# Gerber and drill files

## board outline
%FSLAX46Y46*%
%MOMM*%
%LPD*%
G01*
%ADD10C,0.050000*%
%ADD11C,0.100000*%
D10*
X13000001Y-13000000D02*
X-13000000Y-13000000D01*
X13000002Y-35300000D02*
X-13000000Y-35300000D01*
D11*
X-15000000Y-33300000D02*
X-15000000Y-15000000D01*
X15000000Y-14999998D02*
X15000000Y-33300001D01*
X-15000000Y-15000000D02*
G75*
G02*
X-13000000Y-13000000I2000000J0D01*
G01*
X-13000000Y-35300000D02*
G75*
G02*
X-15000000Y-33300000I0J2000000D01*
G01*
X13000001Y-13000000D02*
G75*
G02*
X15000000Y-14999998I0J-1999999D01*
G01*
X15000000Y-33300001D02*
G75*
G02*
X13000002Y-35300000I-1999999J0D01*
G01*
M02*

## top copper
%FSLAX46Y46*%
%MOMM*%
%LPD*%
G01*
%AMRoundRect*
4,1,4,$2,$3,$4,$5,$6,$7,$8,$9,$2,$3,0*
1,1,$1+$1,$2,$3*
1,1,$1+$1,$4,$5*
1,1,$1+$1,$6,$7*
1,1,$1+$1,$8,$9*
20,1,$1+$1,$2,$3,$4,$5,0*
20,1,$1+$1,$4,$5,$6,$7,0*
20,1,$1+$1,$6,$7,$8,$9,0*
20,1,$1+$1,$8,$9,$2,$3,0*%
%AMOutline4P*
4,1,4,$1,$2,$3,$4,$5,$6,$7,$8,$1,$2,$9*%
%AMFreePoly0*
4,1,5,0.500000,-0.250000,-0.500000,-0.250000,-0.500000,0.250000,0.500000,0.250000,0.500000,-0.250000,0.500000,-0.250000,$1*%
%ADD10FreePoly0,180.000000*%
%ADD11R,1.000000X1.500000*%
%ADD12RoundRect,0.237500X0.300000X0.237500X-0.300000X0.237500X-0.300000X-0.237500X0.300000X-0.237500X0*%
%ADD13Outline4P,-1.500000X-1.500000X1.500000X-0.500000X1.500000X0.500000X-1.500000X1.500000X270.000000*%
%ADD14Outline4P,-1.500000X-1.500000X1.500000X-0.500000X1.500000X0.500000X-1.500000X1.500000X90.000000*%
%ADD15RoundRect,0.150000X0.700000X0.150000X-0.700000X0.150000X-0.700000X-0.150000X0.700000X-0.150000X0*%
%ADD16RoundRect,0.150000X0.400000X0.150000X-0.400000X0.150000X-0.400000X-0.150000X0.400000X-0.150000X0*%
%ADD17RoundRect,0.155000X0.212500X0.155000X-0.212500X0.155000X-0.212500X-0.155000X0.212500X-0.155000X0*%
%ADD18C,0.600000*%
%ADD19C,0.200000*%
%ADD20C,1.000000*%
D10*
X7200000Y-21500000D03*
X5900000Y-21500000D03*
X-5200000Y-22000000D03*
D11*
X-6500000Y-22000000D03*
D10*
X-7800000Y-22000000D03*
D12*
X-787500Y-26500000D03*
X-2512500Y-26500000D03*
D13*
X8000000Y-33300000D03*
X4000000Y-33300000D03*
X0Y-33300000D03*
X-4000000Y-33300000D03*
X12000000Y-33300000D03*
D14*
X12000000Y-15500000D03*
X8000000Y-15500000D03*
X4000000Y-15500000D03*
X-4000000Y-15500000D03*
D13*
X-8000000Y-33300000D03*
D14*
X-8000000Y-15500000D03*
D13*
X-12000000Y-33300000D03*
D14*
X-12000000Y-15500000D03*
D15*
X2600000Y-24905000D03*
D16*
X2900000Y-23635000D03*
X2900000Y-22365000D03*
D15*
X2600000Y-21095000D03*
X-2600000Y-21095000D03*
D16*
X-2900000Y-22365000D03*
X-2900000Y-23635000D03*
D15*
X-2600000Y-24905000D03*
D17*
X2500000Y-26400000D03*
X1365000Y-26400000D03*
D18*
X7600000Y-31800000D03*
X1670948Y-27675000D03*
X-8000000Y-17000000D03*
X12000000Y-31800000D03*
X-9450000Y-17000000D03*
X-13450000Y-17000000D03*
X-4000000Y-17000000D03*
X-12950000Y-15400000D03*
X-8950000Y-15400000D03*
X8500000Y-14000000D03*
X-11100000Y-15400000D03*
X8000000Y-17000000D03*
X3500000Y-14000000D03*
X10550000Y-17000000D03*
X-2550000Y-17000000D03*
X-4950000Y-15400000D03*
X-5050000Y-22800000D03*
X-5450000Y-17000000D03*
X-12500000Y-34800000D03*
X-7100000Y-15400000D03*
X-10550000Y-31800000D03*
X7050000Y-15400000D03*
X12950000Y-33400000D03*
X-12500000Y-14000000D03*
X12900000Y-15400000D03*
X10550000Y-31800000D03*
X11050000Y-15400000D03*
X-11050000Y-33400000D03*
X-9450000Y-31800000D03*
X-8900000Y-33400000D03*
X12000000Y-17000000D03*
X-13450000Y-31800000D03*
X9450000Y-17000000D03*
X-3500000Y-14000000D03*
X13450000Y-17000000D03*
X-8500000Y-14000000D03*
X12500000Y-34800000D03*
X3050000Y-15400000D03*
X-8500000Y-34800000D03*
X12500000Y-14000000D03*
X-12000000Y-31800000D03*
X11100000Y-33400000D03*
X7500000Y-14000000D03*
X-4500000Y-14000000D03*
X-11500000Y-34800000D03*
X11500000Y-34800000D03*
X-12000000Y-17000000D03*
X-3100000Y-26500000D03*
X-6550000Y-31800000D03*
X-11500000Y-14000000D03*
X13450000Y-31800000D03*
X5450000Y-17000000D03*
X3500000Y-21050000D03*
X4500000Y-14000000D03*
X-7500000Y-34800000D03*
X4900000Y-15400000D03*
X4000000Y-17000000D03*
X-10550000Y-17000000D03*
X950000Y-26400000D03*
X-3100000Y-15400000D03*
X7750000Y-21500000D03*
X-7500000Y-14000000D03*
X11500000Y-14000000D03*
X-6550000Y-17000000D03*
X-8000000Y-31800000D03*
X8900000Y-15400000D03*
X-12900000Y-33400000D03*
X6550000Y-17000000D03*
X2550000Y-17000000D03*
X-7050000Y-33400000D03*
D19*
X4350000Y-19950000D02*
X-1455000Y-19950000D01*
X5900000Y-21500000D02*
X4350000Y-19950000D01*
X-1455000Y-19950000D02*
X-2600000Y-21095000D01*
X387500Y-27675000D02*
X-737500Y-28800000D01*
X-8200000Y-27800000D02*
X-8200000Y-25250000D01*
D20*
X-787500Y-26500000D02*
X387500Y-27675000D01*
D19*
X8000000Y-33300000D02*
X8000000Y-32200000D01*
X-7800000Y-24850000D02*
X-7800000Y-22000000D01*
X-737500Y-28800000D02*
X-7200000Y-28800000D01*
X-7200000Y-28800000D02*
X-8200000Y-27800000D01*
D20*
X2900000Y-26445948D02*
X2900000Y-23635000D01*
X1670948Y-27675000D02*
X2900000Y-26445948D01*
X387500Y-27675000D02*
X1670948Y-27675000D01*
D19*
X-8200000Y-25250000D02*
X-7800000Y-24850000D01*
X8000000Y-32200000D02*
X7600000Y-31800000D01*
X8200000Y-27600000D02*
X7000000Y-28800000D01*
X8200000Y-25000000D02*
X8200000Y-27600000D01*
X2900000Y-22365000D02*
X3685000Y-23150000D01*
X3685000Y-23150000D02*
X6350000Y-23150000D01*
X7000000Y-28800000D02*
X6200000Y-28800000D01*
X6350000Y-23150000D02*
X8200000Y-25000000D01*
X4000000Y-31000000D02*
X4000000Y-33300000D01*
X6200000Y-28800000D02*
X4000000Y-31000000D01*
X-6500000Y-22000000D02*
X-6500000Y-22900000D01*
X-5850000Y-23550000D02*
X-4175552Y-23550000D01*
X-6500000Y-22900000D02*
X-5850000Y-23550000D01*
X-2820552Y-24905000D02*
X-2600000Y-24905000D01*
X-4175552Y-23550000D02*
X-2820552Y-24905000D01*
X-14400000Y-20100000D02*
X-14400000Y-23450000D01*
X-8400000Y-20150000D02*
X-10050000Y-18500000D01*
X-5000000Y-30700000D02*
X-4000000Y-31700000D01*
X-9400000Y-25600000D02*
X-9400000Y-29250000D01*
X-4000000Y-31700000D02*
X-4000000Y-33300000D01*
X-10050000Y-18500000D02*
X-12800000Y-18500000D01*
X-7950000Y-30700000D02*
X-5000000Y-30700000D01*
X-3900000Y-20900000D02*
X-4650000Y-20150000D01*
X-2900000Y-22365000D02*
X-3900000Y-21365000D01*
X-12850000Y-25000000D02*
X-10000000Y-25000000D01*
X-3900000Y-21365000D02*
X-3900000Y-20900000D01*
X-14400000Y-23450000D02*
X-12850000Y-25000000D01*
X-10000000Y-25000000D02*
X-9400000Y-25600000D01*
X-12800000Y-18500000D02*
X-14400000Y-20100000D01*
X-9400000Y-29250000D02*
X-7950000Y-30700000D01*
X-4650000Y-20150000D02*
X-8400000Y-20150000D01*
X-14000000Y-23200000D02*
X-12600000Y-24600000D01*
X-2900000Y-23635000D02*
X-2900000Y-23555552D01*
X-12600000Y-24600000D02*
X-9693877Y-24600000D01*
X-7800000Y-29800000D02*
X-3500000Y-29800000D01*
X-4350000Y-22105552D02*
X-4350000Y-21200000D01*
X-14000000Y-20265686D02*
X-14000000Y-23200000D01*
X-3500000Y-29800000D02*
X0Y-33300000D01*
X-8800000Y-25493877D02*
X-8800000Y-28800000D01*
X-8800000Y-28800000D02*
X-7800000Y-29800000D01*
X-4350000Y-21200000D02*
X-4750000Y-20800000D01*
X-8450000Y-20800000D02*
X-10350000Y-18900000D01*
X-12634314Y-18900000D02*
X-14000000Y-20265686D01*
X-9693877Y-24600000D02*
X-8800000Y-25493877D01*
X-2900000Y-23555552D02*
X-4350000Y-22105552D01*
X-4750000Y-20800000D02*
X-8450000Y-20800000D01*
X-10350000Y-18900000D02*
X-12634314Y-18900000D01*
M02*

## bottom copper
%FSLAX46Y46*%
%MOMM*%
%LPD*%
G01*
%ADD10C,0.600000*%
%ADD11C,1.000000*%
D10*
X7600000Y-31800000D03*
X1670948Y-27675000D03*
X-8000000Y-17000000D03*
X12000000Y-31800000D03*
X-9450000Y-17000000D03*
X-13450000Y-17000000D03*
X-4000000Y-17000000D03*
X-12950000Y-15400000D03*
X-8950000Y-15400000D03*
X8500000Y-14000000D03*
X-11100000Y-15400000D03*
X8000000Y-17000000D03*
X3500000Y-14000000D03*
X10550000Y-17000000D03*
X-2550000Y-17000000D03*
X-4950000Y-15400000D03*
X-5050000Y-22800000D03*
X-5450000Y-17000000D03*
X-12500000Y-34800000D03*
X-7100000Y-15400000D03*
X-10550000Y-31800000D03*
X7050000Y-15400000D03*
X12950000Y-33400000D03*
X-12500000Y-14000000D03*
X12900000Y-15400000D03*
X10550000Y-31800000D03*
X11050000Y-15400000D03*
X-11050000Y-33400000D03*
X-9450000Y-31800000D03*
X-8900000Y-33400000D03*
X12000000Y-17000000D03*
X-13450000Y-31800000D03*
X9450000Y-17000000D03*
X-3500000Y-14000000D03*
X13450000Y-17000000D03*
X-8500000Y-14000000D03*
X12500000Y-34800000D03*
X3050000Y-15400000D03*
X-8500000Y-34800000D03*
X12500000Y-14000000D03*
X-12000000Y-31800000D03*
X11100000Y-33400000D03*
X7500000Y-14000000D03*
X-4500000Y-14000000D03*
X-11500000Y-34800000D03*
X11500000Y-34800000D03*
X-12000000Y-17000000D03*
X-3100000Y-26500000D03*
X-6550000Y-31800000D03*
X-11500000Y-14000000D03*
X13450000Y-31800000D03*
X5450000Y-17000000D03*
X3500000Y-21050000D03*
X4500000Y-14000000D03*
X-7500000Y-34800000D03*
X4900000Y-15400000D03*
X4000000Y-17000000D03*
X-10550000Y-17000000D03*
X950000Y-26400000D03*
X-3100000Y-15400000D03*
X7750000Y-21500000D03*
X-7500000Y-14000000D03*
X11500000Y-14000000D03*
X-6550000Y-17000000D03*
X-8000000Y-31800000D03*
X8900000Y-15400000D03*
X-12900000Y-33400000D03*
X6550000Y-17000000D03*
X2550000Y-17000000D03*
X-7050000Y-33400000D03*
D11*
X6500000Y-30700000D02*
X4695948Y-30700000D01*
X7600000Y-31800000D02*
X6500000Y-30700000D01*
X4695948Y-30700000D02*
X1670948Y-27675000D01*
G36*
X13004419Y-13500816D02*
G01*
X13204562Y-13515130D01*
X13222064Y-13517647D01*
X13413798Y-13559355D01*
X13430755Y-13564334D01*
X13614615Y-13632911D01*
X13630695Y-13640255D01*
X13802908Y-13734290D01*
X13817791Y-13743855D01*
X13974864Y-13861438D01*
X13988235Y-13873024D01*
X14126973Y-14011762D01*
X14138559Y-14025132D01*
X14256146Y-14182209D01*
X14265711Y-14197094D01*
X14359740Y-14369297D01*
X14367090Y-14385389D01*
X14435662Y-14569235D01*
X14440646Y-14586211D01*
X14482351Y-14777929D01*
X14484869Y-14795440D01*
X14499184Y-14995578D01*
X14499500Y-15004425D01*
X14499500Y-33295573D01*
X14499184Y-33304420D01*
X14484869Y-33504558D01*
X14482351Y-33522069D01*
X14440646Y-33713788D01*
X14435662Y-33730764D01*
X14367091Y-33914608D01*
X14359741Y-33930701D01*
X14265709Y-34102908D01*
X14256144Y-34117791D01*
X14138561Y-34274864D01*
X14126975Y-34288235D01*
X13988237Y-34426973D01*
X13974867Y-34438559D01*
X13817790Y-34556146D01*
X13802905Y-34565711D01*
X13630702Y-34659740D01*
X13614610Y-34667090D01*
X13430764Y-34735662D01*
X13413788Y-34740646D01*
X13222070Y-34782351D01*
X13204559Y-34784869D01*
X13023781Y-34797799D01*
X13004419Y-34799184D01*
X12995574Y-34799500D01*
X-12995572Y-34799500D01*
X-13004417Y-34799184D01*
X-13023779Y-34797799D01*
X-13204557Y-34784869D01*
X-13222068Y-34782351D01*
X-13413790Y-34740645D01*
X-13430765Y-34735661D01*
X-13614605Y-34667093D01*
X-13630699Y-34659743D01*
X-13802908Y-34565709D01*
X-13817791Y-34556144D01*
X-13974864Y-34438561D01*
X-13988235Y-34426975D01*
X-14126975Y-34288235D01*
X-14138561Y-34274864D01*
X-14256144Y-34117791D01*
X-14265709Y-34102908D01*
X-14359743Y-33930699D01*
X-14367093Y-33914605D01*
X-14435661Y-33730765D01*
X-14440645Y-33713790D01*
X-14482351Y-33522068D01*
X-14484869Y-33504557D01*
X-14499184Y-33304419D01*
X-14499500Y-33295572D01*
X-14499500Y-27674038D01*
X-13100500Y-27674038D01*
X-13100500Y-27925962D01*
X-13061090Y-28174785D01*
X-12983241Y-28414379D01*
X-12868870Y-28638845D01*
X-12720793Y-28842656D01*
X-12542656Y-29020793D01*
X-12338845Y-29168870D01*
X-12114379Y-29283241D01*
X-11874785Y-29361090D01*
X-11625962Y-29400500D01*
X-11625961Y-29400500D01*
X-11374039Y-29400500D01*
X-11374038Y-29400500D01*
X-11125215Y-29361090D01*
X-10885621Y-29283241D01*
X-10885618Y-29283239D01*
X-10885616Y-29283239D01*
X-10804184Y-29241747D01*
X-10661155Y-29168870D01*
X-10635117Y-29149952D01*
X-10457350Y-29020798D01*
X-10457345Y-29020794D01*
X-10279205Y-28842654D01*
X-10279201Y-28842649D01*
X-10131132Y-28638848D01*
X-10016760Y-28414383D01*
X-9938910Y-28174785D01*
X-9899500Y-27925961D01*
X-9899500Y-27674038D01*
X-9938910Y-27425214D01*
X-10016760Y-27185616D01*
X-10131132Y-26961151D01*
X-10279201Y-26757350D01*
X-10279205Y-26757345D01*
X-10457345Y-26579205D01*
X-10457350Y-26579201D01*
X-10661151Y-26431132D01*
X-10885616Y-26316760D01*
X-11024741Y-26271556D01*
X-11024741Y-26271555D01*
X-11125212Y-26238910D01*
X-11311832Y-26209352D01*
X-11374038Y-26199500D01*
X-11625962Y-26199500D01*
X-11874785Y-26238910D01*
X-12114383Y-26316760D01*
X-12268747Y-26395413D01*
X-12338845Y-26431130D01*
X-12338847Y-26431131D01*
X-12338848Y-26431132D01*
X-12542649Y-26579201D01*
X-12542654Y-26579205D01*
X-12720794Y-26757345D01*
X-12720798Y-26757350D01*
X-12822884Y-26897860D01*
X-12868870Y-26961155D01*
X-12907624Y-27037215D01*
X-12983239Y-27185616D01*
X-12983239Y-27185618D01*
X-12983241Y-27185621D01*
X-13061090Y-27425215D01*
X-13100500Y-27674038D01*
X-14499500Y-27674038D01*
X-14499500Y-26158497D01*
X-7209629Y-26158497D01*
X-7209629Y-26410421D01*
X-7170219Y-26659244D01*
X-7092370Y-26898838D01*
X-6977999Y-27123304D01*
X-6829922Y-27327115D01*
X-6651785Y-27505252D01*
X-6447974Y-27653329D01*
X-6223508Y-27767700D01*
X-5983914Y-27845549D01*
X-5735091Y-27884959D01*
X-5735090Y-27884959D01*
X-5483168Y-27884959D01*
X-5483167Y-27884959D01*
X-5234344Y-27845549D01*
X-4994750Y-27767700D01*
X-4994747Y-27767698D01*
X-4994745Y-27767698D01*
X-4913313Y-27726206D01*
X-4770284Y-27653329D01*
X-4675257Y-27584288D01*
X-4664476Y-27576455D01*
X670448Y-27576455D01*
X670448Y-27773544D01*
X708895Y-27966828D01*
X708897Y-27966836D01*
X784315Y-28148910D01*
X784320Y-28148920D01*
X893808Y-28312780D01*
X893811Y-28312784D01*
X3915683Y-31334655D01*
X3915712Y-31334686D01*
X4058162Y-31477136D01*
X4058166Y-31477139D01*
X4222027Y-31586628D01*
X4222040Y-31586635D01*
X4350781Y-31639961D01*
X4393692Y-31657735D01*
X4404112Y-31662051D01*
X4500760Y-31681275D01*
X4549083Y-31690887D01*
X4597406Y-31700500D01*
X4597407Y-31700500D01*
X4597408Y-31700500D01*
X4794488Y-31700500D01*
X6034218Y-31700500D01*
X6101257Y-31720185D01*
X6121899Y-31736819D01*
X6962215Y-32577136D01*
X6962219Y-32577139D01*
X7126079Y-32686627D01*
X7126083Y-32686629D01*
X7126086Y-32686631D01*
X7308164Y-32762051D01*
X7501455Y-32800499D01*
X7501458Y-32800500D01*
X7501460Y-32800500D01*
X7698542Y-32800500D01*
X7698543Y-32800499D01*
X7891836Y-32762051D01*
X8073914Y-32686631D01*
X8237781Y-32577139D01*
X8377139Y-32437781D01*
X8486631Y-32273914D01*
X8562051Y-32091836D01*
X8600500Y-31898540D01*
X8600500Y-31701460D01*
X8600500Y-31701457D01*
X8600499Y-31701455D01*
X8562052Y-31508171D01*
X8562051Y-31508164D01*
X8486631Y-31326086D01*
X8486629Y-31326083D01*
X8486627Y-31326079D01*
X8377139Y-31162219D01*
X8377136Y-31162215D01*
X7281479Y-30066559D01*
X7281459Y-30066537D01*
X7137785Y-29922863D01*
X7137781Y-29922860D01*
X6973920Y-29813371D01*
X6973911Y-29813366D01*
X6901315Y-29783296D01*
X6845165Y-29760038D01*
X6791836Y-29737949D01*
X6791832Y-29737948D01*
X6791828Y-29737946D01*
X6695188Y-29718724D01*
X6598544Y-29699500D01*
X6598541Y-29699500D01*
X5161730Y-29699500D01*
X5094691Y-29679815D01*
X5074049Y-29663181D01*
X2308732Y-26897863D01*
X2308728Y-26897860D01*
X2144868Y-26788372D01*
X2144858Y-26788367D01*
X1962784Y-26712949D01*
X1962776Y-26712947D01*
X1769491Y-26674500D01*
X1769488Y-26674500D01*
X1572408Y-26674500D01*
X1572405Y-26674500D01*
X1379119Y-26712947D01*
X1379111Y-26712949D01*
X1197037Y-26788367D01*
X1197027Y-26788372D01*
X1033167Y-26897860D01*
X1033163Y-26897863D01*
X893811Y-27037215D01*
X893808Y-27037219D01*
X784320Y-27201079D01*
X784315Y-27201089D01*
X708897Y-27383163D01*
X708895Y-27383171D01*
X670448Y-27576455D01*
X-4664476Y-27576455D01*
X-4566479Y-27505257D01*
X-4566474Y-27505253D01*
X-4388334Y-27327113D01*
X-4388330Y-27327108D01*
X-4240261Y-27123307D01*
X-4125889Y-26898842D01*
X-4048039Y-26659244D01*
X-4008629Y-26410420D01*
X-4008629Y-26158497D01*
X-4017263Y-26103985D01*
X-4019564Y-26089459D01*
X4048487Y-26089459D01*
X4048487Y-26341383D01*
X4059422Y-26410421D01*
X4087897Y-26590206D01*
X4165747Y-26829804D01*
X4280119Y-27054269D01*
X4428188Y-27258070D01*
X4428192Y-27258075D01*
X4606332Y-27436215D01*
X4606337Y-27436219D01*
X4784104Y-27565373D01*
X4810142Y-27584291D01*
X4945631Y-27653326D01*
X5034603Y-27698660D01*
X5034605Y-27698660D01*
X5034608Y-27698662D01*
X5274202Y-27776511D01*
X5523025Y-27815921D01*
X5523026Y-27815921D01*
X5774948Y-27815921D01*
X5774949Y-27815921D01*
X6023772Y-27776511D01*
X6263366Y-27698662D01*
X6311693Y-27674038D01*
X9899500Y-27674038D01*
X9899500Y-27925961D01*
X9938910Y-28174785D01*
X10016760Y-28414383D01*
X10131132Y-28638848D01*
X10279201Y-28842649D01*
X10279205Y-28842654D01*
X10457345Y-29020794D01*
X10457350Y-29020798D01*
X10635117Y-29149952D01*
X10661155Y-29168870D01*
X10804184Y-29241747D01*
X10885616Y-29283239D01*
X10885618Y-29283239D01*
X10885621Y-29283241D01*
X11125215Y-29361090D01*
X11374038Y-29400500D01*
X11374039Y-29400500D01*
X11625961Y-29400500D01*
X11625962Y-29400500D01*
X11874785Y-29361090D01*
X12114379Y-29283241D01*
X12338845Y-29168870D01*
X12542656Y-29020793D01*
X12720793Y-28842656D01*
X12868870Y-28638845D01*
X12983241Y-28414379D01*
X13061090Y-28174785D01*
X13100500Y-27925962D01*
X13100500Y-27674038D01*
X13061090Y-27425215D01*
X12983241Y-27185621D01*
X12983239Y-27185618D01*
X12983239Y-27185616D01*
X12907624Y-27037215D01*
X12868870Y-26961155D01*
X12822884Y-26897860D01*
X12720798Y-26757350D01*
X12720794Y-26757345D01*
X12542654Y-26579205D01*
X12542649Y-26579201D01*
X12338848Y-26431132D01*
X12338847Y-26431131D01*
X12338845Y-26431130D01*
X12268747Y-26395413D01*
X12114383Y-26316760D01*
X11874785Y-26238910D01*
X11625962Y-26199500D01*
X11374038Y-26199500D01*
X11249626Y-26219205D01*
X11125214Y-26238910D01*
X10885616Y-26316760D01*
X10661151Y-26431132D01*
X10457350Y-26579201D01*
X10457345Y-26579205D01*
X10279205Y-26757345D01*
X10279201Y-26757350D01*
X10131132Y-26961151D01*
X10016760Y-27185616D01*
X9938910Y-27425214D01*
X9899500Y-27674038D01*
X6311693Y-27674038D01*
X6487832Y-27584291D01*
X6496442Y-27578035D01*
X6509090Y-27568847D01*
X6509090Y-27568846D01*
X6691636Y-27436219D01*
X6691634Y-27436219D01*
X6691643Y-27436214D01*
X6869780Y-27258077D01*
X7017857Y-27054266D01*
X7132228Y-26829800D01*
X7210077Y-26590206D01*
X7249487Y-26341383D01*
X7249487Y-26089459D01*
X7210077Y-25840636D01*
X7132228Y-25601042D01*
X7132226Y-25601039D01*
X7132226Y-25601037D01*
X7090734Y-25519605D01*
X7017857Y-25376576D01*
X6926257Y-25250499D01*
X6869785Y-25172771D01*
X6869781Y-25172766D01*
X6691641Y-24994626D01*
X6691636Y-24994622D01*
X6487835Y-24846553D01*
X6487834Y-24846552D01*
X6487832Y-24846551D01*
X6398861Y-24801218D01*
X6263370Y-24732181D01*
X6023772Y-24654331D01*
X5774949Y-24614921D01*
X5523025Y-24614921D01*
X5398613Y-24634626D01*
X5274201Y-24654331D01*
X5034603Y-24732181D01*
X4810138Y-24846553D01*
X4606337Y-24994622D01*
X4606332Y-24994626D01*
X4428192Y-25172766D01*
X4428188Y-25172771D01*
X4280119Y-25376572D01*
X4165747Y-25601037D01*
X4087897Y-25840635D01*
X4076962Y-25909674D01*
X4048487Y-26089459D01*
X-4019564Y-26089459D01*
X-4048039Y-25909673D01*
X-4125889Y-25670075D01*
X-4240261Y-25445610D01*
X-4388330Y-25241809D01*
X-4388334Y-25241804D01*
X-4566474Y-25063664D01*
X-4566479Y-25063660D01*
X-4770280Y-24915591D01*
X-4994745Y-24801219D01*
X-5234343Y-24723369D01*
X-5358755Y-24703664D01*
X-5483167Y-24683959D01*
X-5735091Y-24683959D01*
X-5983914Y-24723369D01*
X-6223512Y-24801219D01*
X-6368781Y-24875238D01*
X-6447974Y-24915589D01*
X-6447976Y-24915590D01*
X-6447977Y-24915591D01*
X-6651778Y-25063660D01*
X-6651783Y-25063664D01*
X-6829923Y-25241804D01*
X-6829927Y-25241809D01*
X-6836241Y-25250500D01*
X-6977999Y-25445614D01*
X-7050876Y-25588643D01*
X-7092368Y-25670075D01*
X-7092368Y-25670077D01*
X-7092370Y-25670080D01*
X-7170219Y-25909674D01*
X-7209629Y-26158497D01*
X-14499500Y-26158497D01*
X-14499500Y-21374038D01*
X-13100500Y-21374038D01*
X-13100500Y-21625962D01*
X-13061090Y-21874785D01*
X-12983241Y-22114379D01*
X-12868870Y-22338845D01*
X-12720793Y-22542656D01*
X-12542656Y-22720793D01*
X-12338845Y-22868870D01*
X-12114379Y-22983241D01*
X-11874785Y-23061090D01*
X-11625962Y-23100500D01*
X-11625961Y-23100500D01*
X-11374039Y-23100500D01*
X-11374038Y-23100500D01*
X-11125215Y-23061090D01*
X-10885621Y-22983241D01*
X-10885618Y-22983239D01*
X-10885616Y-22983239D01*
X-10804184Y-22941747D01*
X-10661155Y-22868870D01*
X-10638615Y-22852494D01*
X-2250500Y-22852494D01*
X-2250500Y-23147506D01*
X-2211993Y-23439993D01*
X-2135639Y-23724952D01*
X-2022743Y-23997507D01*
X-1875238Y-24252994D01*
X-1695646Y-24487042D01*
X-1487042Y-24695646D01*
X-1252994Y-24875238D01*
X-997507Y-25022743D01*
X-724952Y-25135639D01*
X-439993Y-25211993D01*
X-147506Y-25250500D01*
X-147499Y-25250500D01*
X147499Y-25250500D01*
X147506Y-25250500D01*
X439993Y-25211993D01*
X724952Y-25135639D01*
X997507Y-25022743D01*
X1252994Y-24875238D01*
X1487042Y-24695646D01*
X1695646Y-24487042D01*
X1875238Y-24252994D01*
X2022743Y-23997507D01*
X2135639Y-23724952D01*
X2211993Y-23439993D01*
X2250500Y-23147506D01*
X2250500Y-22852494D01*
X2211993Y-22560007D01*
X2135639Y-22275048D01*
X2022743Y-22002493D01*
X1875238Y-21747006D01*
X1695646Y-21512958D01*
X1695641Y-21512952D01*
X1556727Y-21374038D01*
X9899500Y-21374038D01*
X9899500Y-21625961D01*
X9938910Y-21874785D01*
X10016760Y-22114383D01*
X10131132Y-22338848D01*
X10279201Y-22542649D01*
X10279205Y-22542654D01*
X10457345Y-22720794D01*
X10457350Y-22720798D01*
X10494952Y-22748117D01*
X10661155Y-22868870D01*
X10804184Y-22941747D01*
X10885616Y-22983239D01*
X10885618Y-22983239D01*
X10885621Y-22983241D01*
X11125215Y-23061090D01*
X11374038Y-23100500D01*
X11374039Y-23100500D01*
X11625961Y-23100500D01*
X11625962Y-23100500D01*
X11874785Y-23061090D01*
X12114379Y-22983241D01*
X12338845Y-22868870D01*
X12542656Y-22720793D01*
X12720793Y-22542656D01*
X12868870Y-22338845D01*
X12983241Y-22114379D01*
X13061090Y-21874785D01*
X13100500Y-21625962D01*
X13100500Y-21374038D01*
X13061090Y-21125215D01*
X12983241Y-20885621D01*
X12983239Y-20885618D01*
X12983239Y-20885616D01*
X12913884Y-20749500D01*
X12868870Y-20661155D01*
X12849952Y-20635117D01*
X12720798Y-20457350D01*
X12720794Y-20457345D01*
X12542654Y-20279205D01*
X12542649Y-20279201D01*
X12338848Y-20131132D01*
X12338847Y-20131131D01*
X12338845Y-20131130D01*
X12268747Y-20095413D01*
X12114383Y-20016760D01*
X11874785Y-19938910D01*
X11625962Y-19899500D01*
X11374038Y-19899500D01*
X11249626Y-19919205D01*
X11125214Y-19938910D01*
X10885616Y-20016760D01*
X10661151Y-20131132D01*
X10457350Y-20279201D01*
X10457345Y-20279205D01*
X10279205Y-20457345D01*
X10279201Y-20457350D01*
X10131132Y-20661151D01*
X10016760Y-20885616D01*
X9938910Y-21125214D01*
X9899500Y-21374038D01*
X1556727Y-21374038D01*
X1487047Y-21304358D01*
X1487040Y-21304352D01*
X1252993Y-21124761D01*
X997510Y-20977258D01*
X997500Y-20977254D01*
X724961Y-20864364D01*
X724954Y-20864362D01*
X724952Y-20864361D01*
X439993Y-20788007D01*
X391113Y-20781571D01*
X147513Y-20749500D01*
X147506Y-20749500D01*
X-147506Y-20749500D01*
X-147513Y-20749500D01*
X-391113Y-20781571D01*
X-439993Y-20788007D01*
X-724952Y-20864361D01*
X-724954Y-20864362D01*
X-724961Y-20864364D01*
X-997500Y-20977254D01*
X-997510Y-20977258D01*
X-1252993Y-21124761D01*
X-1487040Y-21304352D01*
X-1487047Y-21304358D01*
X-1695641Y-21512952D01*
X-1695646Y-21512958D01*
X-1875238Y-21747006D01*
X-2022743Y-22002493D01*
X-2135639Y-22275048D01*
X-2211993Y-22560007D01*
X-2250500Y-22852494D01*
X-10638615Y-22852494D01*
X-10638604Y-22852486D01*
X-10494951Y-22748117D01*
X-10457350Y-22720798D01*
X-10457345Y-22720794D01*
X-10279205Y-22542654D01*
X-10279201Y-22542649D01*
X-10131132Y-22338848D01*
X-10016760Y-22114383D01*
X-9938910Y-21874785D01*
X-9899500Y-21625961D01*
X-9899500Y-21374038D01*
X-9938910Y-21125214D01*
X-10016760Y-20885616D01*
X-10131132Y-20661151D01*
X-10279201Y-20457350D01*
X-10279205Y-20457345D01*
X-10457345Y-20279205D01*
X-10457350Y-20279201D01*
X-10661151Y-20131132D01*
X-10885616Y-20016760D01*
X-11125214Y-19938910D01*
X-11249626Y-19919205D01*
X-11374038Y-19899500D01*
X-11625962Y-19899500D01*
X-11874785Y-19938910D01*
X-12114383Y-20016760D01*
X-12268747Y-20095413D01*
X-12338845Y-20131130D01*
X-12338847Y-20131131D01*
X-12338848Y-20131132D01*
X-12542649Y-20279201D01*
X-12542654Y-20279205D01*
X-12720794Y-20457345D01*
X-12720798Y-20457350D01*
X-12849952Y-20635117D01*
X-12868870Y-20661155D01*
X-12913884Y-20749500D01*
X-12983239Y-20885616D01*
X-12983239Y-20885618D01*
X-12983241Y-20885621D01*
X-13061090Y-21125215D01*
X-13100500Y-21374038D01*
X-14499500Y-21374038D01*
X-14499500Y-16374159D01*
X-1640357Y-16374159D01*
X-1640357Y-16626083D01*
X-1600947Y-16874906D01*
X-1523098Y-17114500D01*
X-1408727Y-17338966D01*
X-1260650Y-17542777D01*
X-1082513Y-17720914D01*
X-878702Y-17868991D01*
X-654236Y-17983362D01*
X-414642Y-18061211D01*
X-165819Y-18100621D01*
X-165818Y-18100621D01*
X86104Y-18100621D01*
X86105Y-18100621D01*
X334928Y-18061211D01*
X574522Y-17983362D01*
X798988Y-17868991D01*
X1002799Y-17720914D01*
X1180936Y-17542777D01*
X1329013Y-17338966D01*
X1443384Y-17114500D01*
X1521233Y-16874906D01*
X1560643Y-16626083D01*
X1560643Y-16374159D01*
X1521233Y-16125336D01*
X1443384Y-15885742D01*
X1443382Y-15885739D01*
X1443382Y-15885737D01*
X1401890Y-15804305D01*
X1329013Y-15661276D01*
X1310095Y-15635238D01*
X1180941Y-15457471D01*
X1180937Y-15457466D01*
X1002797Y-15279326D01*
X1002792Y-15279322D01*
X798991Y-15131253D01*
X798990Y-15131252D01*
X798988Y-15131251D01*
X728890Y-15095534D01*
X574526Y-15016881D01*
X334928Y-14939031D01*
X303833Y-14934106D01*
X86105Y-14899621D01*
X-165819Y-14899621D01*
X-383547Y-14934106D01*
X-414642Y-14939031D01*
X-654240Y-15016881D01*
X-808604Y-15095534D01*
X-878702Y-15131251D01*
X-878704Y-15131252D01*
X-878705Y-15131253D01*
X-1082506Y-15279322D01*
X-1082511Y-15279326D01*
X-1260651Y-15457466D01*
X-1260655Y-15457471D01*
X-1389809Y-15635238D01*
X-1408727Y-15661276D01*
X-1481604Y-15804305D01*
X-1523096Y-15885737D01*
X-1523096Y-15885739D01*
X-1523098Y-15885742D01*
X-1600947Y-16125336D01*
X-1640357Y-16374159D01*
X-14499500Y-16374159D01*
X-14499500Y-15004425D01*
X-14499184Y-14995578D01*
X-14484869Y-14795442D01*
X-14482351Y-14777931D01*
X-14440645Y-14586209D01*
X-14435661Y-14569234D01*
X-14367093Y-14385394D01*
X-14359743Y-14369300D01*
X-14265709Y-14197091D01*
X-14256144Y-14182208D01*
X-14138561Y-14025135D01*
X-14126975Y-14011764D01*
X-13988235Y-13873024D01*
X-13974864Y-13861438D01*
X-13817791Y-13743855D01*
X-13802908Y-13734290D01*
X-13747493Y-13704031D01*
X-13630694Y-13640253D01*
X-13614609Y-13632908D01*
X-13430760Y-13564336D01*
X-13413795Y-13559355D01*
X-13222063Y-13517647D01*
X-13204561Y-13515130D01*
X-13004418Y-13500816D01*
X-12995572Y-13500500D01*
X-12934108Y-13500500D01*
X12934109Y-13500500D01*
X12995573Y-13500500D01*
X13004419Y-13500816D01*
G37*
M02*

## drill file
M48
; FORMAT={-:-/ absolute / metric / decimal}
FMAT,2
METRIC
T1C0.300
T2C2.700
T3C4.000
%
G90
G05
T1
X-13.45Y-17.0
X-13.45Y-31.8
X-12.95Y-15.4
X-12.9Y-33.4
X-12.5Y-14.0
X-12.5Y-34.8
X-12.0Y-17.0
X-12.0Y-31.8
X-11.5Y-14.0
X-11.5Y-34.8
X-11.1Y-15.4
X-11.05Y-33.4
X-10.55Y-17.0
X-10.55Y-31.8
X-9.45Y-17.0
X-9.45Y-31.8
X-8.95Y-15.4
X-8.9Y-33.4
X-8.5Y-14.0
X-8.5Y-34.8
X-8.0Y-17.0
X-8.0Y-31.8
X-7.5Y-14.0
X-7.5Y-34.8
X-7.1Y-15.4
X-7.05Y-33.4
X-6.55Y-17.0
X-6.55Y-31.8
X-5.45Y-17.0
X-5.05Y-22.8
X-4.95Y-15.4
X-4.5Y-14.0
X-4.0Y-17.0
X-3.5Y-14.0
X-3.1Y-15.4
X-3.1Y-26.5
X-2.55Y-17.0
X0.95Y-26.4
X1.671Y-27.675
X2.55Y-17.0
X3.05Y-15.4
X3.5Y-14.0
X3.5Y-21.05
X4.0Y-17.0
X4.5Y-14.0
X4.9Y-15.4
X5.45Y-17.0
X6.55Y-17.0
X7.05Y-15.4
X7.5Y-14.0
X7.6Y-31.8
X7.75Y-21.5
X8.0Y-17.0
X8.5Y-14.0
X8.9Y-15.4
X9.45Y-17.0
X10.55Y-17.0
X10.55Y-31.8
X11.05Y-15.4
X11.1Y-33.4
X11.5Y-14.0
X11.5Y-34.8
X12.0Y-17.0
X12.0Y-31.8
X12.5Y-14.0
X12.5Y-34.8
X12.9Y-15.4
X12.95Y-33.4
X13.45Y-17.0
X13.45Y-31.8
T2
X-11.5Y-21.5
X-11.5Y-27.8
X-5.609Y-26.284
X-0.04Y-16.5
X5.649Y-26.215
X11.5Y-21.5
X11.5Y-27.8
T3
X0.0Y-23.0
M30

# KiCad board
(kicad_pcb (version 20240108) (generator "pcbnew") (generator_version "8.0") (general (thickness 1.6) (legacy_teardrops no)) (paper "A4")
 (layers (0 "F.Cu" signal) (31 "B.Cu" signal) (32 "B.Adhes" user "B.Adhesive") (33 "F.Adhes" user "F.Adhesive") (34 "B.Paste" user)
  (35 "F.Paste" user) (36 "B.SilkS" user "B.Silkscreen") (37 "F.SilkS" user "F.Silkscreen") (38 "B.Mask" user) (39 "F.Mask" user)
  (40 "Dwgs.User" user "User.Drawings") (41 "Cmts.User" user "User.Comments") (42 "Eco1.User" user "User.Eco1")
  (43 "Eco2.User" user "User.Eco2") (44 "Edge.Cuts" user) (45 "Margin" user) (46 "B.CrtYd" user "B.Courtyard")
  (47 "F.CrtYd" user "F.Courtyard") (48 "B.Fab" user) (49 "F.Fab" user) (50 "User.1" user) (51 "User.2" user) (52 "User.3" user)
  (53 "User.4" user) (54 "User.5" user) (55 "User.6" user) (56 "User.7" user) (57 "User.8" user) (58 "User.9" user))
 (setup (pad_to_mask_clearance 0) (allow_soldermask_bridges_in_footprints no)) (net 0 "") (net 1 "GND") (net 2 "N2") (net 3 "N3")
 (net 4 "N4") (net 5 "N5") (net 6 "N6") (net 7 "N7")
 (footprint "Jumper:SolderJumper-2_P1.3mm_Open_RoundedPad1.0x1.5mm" (layer "F.Cu") (at 6.55 21.5 180)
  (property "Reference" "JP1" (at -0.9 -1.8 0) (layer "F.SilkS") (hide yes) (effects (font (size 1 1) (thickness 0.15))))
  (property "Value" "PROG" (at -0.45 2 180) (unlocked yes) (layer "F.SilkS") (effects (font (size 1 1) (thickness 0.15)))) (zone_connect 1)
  (pad "1" smd custom (at -0.65 0 180) (size 1 0.5) (layers "F.Cu" "F.Mask") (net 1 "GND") (zone_connect 2) (thermal_bridge_angle 45)
   (options (clearance outline) (anchor rect)) (primitives))
  (pad "2" smd custom (at 0.65 0 180) (size 1 0.5) (layers "F.Cu" "F.Mask") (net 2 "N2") (zone_connect 2) (thermal_bridge_angle 45)
   (options (clearance outline) (anchor rect)) (primitives)))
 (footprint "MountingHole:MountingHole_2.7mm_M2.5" (layer "F.Cu") (at -11.5 21.5 180)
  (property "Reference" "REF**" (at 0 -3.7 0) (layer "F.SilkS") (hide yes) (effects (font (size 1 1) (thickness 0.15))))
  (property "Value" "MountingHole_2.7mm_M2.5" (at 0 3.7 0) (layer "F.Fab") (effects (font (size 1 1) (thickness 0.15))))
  (pad "" np_thru_hole circle (at 0 0 180) (size 2.7 2.7) (drill 2.7) (layers "*.Cu" "*.Mask")))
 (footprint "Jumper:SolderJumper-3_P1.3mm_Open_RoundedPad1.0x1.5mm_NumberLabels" (layer "F.Cu") (at -6.5 22 180)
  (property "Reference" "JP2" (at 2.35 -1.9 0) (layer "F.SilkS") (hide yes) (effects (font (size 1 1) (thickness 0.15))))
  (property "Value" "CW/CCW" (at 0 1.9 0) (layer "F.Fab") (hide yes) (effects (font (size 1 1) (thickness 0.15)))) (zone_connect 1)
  (pad "1" smd custom (at -1.3 0 180) (size 1 0.5) (layers "F.Cu" "F.Mask") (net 1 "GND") (zone_connect 2) (thermal_bridge_angle 45)
   (options (clearance outline) (anchor rect)) (primitives))
  (pad "2" smd rect (at 0 0 180) (size 1 1.5) (layers "F.Cu" "F.Mask") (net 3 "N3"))
  (pad "3" smd custom (at 1.3 0 180) (size 1 0.5) (layers "F.Cu" "F.Mask") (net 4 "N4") (zone_connect 2) (thermal_bridge_angle 45)
   (options (clearance outline) (anchor rect)) (primitives)))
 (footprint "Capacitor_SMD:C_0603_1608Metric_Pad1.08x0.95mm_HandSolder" (layer "F.Cu") (at -1.65 26.5 180)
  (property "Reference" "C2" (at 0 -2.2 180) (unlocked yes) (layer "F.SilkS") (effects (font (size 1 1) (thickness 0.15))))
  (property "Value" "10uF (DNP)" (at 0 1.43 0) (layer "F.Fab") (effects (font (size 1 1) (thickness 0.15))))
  (pad "1" smd roundrect (at -0.8625 0 180) (size 1.075 0.95) (layers "F.Cu" "F.Paste" "F.Mask") (roundrect_rratio 0.25) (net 4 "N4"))
  (pad "2" smd roundrect (at 0.8625 0 180) (size 1.075 0.95) (layers "F.Cu" "F.Paste" "F.Mask") (roundrect_rratio 0.25) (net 1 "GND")))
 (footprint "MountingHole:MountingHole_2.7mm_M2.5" (layer "F.Cu") (at 11.5 21.5 180)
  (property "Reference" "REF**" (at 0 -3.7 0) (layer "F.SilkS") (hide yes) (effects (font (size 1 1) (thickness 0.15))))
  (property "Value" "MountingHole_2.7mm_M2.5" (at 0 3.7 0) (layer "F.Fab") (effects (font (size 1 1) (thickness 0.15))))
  (pad "" np_thru_hole circle (at 0 0 180) (size 2.7 2.7) (drill 2.7) (layers "*.Cu" "*.Mask")))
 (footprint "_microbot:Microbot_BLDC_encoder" (layer "F.Cu") (at 0 23 180)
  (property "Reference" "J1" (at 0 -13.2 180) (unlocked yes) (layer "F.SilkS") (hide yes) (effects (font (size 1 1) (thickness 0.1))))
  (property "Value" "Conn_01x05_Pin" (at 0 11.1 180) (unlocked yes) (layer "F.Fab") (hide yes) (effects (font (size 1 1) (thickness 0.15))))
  (fp_line (start 15 -10.3) (end 15 8) (stroke (width 0.1) (type default)) (layer "Edge.Cuts"))
  (fp_line (start -15 8.000002) (end -15 -10.300001) (stroke (width 0.1) (type default)) (layer "Edge.Cuts"))
  (fp_arc (start 15 8) (mid 14.414214 9.414214) (end 13 10) (stroke (width 0.1) (type default)) (layer "Edge.Cuts"))
  (fp_arc (start 13 -12.3) (mid 14.414214 -11.714214) (end 15 -10.3) (stroke (width 0.1) (type default)) (layer "Edge.Cuts"))
  (fp_arc (start -13.000001 10) (mid -14.414214 9.414214) (end -15 8.000002) (stroke (width 0.1) (type default)) (layer "Edge.Cuts"))
  (fp_arc (start -15 -10.300001) (mid -14.414214 -11.714214) (end -13.000002 -12.3) (stroke (width 0.1) (type default)) (layer "Edge.Cuts"))
  (pad "" np_thru_hole circle (at -5.648987 -3.215421 270) (size 2.7 2.7) (drill 2.7) (layers "F&B.Cu" "*.Mask"))
  (pad "" np_thru_hole circle (at 0 0 270) (size 4 4) (drill 4) (layers "F&B.Cu" "*.Mask"))
  (pad "" np_thru_hole circle (at 0.039857 6.499879 270) (size 2.7 2.7) (drill 2.7) (layers "F&B.Cu" "*.Mask"))
  (pad "" np_thru_hole circle (at 5.609129 -3.284459 270) (size 2.7 2.7) (drill 2.7) (layers "F&B.Cu" "*.Mask"))
  (pad "1" smd trapezoid (at -8 -10.3 270) (size 3 2) (rect_delta 1 0) (layers "F.Cu" "F.Paste" "F.Mask") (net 4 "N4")
   (thermal_bridge_angle 45))
  (pad "2" smd trapezoid (at -4 -10.3 270) (size 3 2) (rect_delta 1 0) (layers "F.Cu" "F.Paste" "F.Mask") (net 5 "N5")
   (thermal_bridge_angle 45))
  (pad "3" smd trapezoid (at 0 -10.3 270) (size 3 2) (rect_delta 1 0) (layers "F.Cu" "F.Paste" "F.Mask") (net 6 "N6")
   (thermal_bridge_angle 45))
  (pad "4" smd trapezoid (at 4 -10.3 270) (size 3 2) (rect_delta 1 0) (layers "F.Cu" "F.Paste" "F.Mask") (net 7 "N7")
   (thermal_bridge_angle 45))
  (pad "5" smd trapezoid (at -12 -10.3 270) (size 3 2) (rect_delta 1 0) (layers "F.Cu" "F.Paste" "F.Mask") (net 1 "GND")
   (thermal_bridge_angle 45))
  (pad "5" smd trapezoid (at -12 7.5 90) (size 3 2) (rect_delta 1 0) (layers "F.Cu" "F.Paste" "F.Mask") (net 1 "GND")
   (thermal_bridge_angle 45))
  (pad "5" smd trapezoid (at -8 7.5 90) (size 3 2) (rect_delta 1 0) (layers "F.Cu" "F.Paste" "F.Mask") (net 1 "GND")
   (thermal_bridge_angle 45))
  (pad "5" smd trapezoid (at -4 7.5 90) (size 3 2) (rect_delta 1 0) (layers "F.Cu" "F.Paste" "F.Mask") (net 1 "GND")
   (thermal_bridge_angle 45))
  (pad "5" smd trapezoid (at 4 7.5 90) (size 3 2) (rect_delta 1 0) (layers "F.Cu" "F.Paste" "F.Mask") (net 1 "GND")
   (thermal_bridge_angle 45))
  (pad "5" smd trapezoid (at 8 -10.3 270) (size 3 2) (rect_delta 1 0) (layers "F.Cu" "F.Paste" "F.Mask") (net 1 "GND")
   (thermal_bridge_angle 45))
  (pad "5" smd trapezoid (at 8 7.5 90) (size 3 2) (rect_delta 1 0) (layers "F.Cu" "F.Paste" "F.Mask") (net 1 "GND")
   (thermal_bridge_angle 45))
  (pad "5" smd trapezoid (at 12 -10.3 270) (size 3 2) (rect_delta 1 0) (layers "F.Cu" "F.Paste" "F.Mask") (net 1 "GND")
   (thermal_bridge_angle 45))
  (pad "5" smd trapezoid (at 12 7.5 90) (size 3 2) (rect_delta 1 0) (layers "F.Cu" "F.Paste" "F.Mask") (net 1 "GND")
   (thermal_bridge_angle 45)))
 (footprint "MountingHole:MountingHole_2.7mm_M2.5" (layer "F.Cu") (at 11.5 27.8 180)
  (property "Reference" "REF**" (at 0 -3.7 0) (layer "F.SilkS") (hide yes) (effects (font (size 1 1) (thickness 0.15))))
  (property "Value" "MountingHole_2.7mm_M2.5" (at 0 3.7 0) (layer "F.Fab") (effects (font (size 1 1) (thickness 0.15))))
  (pad "" np_thru_hole circle (at 0 0 180) (size 2.7 2.7) (drill 2.7) (layers "*.Cu" "*.Mask")))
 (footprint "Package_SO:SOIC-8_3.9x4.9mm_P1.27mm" (layer "F.Cu") (at 0 23 180)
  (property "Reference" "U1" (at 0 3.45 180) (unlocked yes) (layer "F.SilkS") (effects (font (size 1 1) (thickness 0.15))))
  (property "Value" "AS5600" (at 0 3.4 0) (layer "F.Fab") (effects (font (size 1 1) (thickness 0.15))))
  (pad "1" smd roundrect (at -2.6 -1.905 180) (size 1.7 0.6) (layers "F.Cu" "F.Paste" "F.Mask") (roundrect_rratio 0.25) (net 4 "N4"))
  (pad "2" smd roundrect (at -2.9 -0.635 180) (size 1.1 0.6) (layers "F.Cu" "F.Paste" "F.Mask") (roundrect_rratio 0.25) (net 4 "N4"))
  (pad "3" smd roundrect (at -2.9 0.635 180) (size 1.1 0.6) (layers "F.Cu" "F.Paste" "F.Mask") (roundrect_rratio 0.25) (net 5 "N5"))
  (pad "4" smd roundrect (at -2.6 1.905 180) (size 1.7 0.6) (layers "F.Cu" "F.Paste" "F.Mask") (roundrect_rratio 0.25) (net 1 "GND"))
  (pad "5" smd roundrect (at 2.6 1.905 180) (size 1.7 0.6) (layers "F.Cu" "F.Paste" "F.Mask") (roundrect_rratio 0.25) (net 2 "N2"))
  (pad "6" smd roundrect (at 2.9 0.635 180) (size 1.1 0.6) (layers "F.Cu" "F.Paste" "F.Mask") (roundrect_rratio 0.25) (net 7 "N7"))
  (pad "7" smd roundrect (at 2.9 -0.635 180) (size 1.1 0.6) (layers "F.Cu" "F.Paste" "F.Mask") (roundrect_rratio 0.25) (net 6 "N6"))
  (pad "8" smd roundrect (at 2.6 -1.905 180) (size 1.7 0.6) (layers "F.Cu" "F.Paste" "F.Mask") (roundrect_rratio 0.25) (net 3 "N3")))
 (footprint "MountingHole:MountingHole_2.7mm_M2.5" (layer "F.Cu") (at -11.5 27.8 180)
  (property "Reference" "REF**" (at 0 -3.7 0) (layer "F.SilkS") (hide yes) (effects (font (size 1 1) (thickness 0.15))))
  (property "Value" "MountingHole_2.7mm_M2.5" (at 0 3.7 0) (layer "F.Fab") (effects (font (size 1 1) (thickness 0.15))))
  (pad "" np_thru_hole circle (at 0 0 180) (size 2.7 2.7) (drill 2.7) (layers "*.Cu" "*.Mask")))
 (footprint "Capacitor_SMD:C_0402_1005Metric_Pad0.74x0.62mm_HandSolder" (layer "F.Cu") (at 1.9325 26.4 180)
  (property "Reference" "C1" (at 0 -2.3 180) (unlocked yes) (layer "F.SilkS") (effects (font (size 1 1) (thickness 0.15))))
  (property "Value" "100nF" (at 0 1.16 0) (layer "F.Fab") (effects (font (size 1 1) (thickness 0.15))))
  (pad "1" smd roundrect (at -0.5675 0 180) (size 0.735 0.62) (layers "F.Cu" "F.Paste" "F.Mask") (roundrect_rratio 0.25) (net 4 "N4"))
  (pad "2" smd roundrect (at 0.5675 0 180) (size 0.735 0.62) (layers "F.Cu" "F.Paste" "F.Mask") (roundrect_rratio 0.25) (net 1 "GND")))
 (gr_line (start 13.000001 13) (end -13 13) (stroke (width 0.05) (type default)) (layer "Edge.Cuts"))
 (gr_line (start 13.000002 35.3) (end -13 35.3) (stroke (width 0.05) (type default)) (layer "Edge.Cuts"))
 (segment (start 4.35 19.95) (end -1.455 19.95) (width 0.2) (layer "F.Cu") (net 2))
 (segment (start 5.9 21.5) (end 4.35 19.95) (width 0.2) (layer "F.Cu") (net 2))
 (segment (start -1.455 19.95) (end -2.6 21.095) (width 0.2) (layer "F.Cu") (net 2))
 (segment (start 0.3875 27.675) (end -0.7375 28.8) (width 0.2) (layer "F.Cu") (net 4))
 (segment (start -8.2 27.8) (end -8.2 25.25) (width 0.2) (layer "F.Cu") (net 4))
 (segment (start -0.7875 26.5) (end 0.3875 27.675) (width 1) (layer "F.Cu") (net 4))
 (segment (start 8 33.3) (end 8 32.2) (width 0.2) (layer "F.Cu") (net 4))
 (segment (start -7.8 24.85) (end -7.8 22) (width 0.2) (layer "F.Cu") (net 4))
 (segment (start -0.7375 28.8) (end -7.2 28.8) (width 0.2) (layer "F.Cu") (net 4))
 (segment (start -7.2 28.8) (end -8.2 27.8) (width 0.2) (layer "F.Cu") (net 4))
 (segment (start 2.9 26.445948) (end 2.9 23.635) (width 1) (layer "F.Cu") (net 4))
 (segment (start 1.670948 27.675) (end 2.9 26.445948) (width 1) (layer "F.Cu") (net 4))
 (segment (start 0.3875 27.675) (end 1.670948 27.675) (width 1) (layer "F.Cu") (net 4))
 (segment (start -8.2 25.25) (end -7.8 24.85) (width 0.2) (layer "F.Cu") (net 4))
 (segment (start 8 32.2) (end 7.6 31.8) (width 0.2) (layer "F.Cu") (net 4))
 (via (at 7.6 31.8) (size 0.6) (drill 0.3) (layers "F.Cu" "B.Cu") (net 4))
 (via (at 1.670948 27.675) (size 0.6) (drill 0.3) (layers "F.Cu" "B.Cu") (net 4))
 (segment (start 6.5 30.7) (end 4.695948 30.7) (width 1) (layer "B.Cu") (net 4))
 (segment (start 7.6 31.8) (end 6.5 30.7) (width 1) (layer "B.Cu") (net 4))
 (segment (start 4.695948 30.7) (end 1.670948 27.675) (width 1) (layer "B.Cu") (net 4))
 (segment (start 8.2 27.6) (end 7 28.8) (width 0.2) (layer "F.Cu") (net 5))
 (segment (start 8.2 25) (end 8.2 27.6) (width 0.2) (layer "F.Cu") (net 5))
 (segment (start 2.9 22.365) (end 3.685 23.15) (width 0.2) (layer "F.Cu") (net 5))
 (segment (start 3.685 23.15) (end 6.35 23.15) (width 0.2) (layer "F.Cu") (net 5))
 (segment (start 7 28.8) (end 6.2 28.8) (width 0.2) (layer "F.Cu") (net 5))
 (segment (start 6.35 23.15) (end 8.2 25) (width 0.2) (layer "F.Cu") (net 5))
 (segment (start 4 31) (end 4 33.3) (width 0.2) (layer "F.Cu") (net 5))
 (segment (start 6.2 28.8) (end 4 31) (width 0.2) (layer "F.Cu") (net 5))
 (segment (start -6.5 22) (end -6.5 22.9) (width 0.2) (layer "F.Cu") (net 3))
 (segment (start -5.85 23.55) (end -4.175552 23.55) (width 0.2) (layer "F.Cu") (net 3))
 (segment (start -6.5 22.9) (end -5.85 23.55) (width 0.2) (layer "F.Cu") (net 3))
 (segment (start -2.820552 24.905) (end -2.6 24.905) (width 0.2) (layer "F.Cu") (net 3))
 (segment (start -4.175552 23.55) (end -2.820552 24.905) (width 0.2) (layer "F.Cu") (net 3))
 (via (at -8 17) (size 0.6) (drill 0.3) (layers "F.Cu" "B.Cu") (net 1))
 (via (at 12 31.8) (size 0.6) (drill 0.3) (layers "F.Cu" "B.Cu") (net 1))
 (via (at -9.45 17) (size 0.6) (drill 0.3) (layers "F.Cu" "B.Cu") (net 1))
 (via (at -13.45 17) (size 0.6) (drill 0.3) (layers "F.Cu" "B.Cu") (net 1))
 (via (at -4 17) (size 0.6) (drill 0.3) (layers "F.Cu" "B.Cu") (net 1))
 (via (at -12.95 15.4) (size 0.6) (drill 0.3) (layers "F.Cu" "B.Cu") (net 1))
 (via (at -8.95 15.4) (size 0.6) (drill 0.3) (layers "F.Cu" "B.Cu") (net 1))
 (via (at 8.5 14) (size 0.6) (drill 0.3) (layers "F.Cu" "B.Cu") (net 1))
 (via (at -11.1 15.4) (size 0.6) (drill 0.3) (layers "F.Cu" "B.Cu") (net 1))
 (via (at 8 17) (size 0.6) (drill 0.3) (layers "F.Cu" "B.Cu") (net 1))
 (via (at 3.5 14) (size 0.6) (drill 0.3) (layers "F.Cu" "B.Cu") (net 1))
 (via (at 10.55 17) (size 0.6) (drill 0.3) (layers "F.Cu" "B.Cu") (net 1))
 (via (at -2.55 17) (size 0.6) (drill 0.3) (layers "F.Cu" "B.Cu") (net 1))
 (via (at -4.95 15.4) (size 0.6) (drill 0.3) (layers "F.Cu" "B.Cu") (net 1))
 (via (at -5.05 22.8) (size 0.6) (drill 0.3) (layers "F.Cu" "B.Cu") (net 1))
 (via (at -5.45 17) (size 0.6) (drill 0.3) (layers "F.Cu" "B.Cu") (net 1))
 (via (at -12.5 34.8) (size 0.6) (drill 0.3) (layers "F.Cu" "B.Cu") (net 1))
 (via (at -7.1 15.4) (size 0.6) (drill 0.3) (layers "F.Cu" "B.Cu") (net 1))
 (via (at -10.55 31.8) (size 0.6) (drill 0.3) (layers "F.Cu" "B.Cu") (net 1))
 (via (at 7.05 15.4) (size 0.6) (drill 0.3) (layers "F.Cu" "B.Cu") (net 1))
 (via (at 12.95 33.4) (size 0.6) (drill 0.3) (layers "F.Cu" "B.Cu") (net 1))
 (via (at -12.5 14) (size 0.6) (drill 0.3) (layers "F.Cu" "B.Cu") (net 1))
 (via (at 12.9 15.4) (size 0.6) (drill 0.3) (layers "F.Cu" "B.Cu") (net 1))
 (via (at 10.55 31.8) (size 0.6) (drill 0.3) (layers "F.Cu" "B.Cu") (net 1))
 (via (at 11.05 15.4) (size 0.6) (drill 0.3) (layers "F.Cu" "B.Cu") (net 1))
 (via (at -11.05 33.4) (size 0.6) (drill 0.3) (layers "F.Cu" "B.Cu") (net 1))
 (via (at -9.45 31.8) (size 0.6) (drill 0.3) (layers "F.Cu" "B.Cu") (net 1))
 (via (at -8.9 33.4) (size 0.6) (drill 0.3) (layers "F.Cu" "B.Cu") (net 1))
 (via (at 12 17) (size 0.6) (drill 0.3) (layers "F.Cu" "B.Cu") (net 1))
 (via (at -13.45 31.8) (size 0.6) (drill 0.3) (layers "F.Cu" "B.Cu") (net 1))
 (via (at 9.45 17) (size 0.6) (drill 0.3) (layers "F.Cu" "B.Cu") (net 1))
 (via (at -3.5 14) (size 0.6) (drill 0.3) (layers "F.Cu" "B.Cu") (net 1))
 (via (at 13.45 17) (size 0.6) (drill 0.3) (layers "F.Cu" "B.Cu") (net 1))
 (via (at -8.5 14) (size 0.6) (drill 0.3) (layers "F.Cu" "B.Cu") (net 1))
 (via (at 12.5 34.8) (size 0.6) (drill 0.3) (layers "F.Cu" "B.Cu") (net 1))
 (via (at 3.05 15.4) (size 0.6) (drill 0.3) (layers "F.Cu" "B.Cu") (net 1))
 (via (at -8.5 34.8) (size 0.6) (drill 0.3) (layers "F.Cu" "B.Cu") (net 1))
 (via (at 12.5 14) (size 0.6) (drill 0.3) (layers "F.Cu" "B.Cu") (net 1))
 (via (at -12 31.8) (size 0.6) (drill 0.3) (layers "F.Cu" "B.Cu") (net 1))
 (via (at 11.1 33.4) (size 0.6) (drill 0.3) (layers "F.Cu" "B.Cu") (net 1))
 (via (at 7.5 14) (size 0.6) (drill 0.3) (layers "F.Cu" "B.Cu") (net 1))
 (via (at -4.5 14) (size 0.6) (drill 0.3) (layers "F.Cu" "B.Cu") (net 1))
 (via (at -11.5 34.8) (size 0.6) (drill 0.3) (layers "F.Cu" "B.Cu") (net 1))
 (via (at 11.5 34.8) (size 0.6) (drill 0.3) (layers "F.Cu" "B.Cu") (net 1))
 (via (at -12 17) (size 0.6) (drill 0.3) (layers "F.Cu" "B.Cu") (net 1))
 (via (at -3.1 26.5) (size 0.6) (drill 0.3) (layers "F.Cu" "B.Cu") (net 1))
 (via (at -6.55 31.8) (size 0.6) (drill 0.3) (layers "F.Cu" "B.Cu") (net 1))
 (via (at -11.5 14) (size 0.6) (drill 0.3) (layers "F.Cu" "B.Cu") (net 1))
 (via (at 13.45 31.8) (size 0.6) (drill 0.3) (layers "F.Cu" "B.Cu") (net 1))
 (via (at 5.45 17) (size 0.6) (drill 0.3) (layers "F.Cu" "B.Cu") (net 1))
 (via (at 3.5 21.05) (size 0.6) (drill 0.3) (layers "F.Cu" "B.Cu") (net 1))
 (via (at 4.5 14) (size 0.6) (drill 0.3) (layers "F.Cu" "B.Cu") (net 1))
 (via (at -7.5 34.8) (size 0.6) (drill 0.3) (layers "F.Cu" "B.Cu") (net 1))
 (via (at 4.9 15.4) (size 0.6) (drill 0.3) (layers "F.Cu" "B.Cu") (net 1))
 (via (at 4 17) (size 0.6) (drill 0.3) (layers "F.Cu" "B.Cu") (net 1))
 (via (at -10.55 17) (size 0.6) (drill 0.3) (layers "F.Cu" "B.Cu") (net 1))
 (via (at 0.95 26.4) (size 0.6) (drill 0.3) (layers "F.Cu" "B.Cu") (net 1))
 (via (at -3.1 15.4) (size 0.6) (drill 0.3) (layers "F.Cu" "B.Cu") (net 1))
 (via (at 7.75 21.5) (size 0.6) (drill 0.3) (layers "F.Cu" "B.Cu") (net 1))
 (via (at -7.5 14) (size 0.6) (drill 0.3) (layers "F.Cu" "B.Cu") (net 1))
 (via (at 11.5 14) (size 0.6) (drill 0.3) (layers "F.Cu" "B.Cu") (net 1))
 (via (at -6.55 17) (size 0.6) (drill 0.3) (layers "F.Cu" "B.Cu") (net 1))
 (via (at -8 31.8) (size 0.6) (drill 0.3) (layers "F.Cu" "B.Cu") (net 1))
 (via (at 8.9 15.4) (size 0.6) (drill 0.3) (layers "F.Cu" "B.Cu") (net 1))
 (via (at -12.9 33.4) (size 0.6) (drill 0.3) (layers "F.Cu" "B.Cu") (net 1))
 (via (at 6.55 17) (size 0.6) (drill 0.3) (layers "F.Cu" "B.Cu") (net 1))
 (via (at 2.55 17) (size 0.6) (drill 0.3) (layers "F.Cu" "B.Cu") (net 1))
 (via (at -7.05 33.4) (size 0.6) (drill 0.3) (layers "F.Cu" "B.Cu") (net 1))
 (segment (start -14.4 20.1) (end -14.4 23.45) (width 0.2) (layer "F.Cu") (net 7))
 (segment (start -8.4 20.15) (end -10.05 18.5) (width 0.2) (layer "F.Cu") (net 7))
 (segment (start -5 30.7) (end -4 31.7) (width 0.2) (layer "F.Cu") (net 7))
 (segment (start -9.4 25.6) (end -9.4 29.25) (width 0.2) (layer "F.Cu") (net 7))
 (segment (start -4 31.7) (end -4 33.3) (width 0.2) (layer "F.Cu") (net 7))
 (segment (start -10.05 18.5) (end -12.8 18.5) (width 0.2) (layer "F.Cu") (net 7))
 (segment (start -7.95 30.7) (end -5 30.7) (width 0.2) (layer "F.Cu") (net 7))
 (segment (start -3.9 20.9) (end -4.65 20.15) (width 0.2) (layer "F.Cu") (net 7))
 (segment (start -2.9 22.365) (end -3.9 21.365) (width 0.2) (layer "F.Cu") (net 7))
 (segment (start -12.85 25) (end -10 25) (width 0.2) (layer "F.Cu") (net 7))
 (segment (start -3.9 21.365) (end -3.9 20.9) (width 0.2) (layer "F.Cu") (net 7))
 (segment (start -14.4 23.45) (end -12.85 25) (width 0.2) (layer "F.Cu") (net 7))
 (segment (start -10 25) (end -9.4 25.6) (width 0.2) (layer "F.Cu") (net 7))
 (segment (start -12.8 18.5) (end -14.4 20.1) (width 0.2) (layer "F.Cu") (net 7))
 (segment (start -9.4 29.25) (end -7.95 30.7) (width 0.2) (layer "F.Cu") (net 7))
 (segment (start -4.65 20.15) (end -8.4 20.15) (width 0.2) (layer "F.Cu") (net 7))
 (segment (start -14 23.2) (end -12.6 24.6) (width 0.2) (layer "F.Cu") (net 6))
 (segment (start -2.9 23.635) (end -2.9 23.555552) (width 0.2) (layer "F.Cu") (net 6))
 (segment (start -12.6 24.6) (end -9.693877 24.6) (width 0.2) (layer "F.Cu") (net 6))
 (segment (start -7.8 29.8) (end -3.5 29.8) (width 0.2) (layer "F.Cu") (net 6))
 (segment (start -4.35 22.105552) (end -4.35 21.2) (width 0.2) (layer "F.Cu") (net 6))
 (segment (start -14 20.265686) (end -14 23.2) (width 0.2) (layer "F.Cu") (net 6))
 (segment (start -3.5 29.8) (end 0 33.3) (width 0.2) (layer "F.Cu") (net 6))
 (segment (start -8.8 25.493877) (end -8.8 28.8) (width 0.2) (layer "F.Cu") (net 6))
 (segment (start -8.8 28.8) (end -7.8 29.8) (width 0.2) (layer "F.Cu") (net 6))
 (segment (start -4.35 21.2) (end -4.75 20.8) (width 0.2) (layer "F.Cu") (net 6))
 (segment (start -8.45 20.8) (end -10.35 18.9) (width 0.2) (layer "F.Cu") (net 6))
 (segment (start -12.634314 18.9) (end -14 20.265686) (width 0.2) (layer "F.Cu") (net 6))
 (segment (start -9.693877 24.6) (end -8.8 25.493877) (width 0.2) (layer "F.Cu") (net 6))
 (segment (start -2.9 23.555552) (end -4.35 22.105552) (width 0.2) (layer "F.Cu") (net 6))
 (segment (start -4.75 20.8) (end -8.45 20.8) (width 0.2) (layer "F.Cu") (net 6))
 (segment (start -10.35 18.9) (end -12.634314 18.9) (width 0.2) (layer "F.Cu") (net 6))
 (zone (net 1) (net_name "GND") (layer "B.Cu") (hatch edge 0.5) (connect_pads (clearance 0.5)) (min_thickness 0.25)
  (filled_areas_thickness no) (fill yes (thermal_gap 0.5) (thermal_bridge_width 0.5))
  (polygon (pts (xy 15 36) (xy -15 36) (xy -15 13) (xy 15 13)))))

